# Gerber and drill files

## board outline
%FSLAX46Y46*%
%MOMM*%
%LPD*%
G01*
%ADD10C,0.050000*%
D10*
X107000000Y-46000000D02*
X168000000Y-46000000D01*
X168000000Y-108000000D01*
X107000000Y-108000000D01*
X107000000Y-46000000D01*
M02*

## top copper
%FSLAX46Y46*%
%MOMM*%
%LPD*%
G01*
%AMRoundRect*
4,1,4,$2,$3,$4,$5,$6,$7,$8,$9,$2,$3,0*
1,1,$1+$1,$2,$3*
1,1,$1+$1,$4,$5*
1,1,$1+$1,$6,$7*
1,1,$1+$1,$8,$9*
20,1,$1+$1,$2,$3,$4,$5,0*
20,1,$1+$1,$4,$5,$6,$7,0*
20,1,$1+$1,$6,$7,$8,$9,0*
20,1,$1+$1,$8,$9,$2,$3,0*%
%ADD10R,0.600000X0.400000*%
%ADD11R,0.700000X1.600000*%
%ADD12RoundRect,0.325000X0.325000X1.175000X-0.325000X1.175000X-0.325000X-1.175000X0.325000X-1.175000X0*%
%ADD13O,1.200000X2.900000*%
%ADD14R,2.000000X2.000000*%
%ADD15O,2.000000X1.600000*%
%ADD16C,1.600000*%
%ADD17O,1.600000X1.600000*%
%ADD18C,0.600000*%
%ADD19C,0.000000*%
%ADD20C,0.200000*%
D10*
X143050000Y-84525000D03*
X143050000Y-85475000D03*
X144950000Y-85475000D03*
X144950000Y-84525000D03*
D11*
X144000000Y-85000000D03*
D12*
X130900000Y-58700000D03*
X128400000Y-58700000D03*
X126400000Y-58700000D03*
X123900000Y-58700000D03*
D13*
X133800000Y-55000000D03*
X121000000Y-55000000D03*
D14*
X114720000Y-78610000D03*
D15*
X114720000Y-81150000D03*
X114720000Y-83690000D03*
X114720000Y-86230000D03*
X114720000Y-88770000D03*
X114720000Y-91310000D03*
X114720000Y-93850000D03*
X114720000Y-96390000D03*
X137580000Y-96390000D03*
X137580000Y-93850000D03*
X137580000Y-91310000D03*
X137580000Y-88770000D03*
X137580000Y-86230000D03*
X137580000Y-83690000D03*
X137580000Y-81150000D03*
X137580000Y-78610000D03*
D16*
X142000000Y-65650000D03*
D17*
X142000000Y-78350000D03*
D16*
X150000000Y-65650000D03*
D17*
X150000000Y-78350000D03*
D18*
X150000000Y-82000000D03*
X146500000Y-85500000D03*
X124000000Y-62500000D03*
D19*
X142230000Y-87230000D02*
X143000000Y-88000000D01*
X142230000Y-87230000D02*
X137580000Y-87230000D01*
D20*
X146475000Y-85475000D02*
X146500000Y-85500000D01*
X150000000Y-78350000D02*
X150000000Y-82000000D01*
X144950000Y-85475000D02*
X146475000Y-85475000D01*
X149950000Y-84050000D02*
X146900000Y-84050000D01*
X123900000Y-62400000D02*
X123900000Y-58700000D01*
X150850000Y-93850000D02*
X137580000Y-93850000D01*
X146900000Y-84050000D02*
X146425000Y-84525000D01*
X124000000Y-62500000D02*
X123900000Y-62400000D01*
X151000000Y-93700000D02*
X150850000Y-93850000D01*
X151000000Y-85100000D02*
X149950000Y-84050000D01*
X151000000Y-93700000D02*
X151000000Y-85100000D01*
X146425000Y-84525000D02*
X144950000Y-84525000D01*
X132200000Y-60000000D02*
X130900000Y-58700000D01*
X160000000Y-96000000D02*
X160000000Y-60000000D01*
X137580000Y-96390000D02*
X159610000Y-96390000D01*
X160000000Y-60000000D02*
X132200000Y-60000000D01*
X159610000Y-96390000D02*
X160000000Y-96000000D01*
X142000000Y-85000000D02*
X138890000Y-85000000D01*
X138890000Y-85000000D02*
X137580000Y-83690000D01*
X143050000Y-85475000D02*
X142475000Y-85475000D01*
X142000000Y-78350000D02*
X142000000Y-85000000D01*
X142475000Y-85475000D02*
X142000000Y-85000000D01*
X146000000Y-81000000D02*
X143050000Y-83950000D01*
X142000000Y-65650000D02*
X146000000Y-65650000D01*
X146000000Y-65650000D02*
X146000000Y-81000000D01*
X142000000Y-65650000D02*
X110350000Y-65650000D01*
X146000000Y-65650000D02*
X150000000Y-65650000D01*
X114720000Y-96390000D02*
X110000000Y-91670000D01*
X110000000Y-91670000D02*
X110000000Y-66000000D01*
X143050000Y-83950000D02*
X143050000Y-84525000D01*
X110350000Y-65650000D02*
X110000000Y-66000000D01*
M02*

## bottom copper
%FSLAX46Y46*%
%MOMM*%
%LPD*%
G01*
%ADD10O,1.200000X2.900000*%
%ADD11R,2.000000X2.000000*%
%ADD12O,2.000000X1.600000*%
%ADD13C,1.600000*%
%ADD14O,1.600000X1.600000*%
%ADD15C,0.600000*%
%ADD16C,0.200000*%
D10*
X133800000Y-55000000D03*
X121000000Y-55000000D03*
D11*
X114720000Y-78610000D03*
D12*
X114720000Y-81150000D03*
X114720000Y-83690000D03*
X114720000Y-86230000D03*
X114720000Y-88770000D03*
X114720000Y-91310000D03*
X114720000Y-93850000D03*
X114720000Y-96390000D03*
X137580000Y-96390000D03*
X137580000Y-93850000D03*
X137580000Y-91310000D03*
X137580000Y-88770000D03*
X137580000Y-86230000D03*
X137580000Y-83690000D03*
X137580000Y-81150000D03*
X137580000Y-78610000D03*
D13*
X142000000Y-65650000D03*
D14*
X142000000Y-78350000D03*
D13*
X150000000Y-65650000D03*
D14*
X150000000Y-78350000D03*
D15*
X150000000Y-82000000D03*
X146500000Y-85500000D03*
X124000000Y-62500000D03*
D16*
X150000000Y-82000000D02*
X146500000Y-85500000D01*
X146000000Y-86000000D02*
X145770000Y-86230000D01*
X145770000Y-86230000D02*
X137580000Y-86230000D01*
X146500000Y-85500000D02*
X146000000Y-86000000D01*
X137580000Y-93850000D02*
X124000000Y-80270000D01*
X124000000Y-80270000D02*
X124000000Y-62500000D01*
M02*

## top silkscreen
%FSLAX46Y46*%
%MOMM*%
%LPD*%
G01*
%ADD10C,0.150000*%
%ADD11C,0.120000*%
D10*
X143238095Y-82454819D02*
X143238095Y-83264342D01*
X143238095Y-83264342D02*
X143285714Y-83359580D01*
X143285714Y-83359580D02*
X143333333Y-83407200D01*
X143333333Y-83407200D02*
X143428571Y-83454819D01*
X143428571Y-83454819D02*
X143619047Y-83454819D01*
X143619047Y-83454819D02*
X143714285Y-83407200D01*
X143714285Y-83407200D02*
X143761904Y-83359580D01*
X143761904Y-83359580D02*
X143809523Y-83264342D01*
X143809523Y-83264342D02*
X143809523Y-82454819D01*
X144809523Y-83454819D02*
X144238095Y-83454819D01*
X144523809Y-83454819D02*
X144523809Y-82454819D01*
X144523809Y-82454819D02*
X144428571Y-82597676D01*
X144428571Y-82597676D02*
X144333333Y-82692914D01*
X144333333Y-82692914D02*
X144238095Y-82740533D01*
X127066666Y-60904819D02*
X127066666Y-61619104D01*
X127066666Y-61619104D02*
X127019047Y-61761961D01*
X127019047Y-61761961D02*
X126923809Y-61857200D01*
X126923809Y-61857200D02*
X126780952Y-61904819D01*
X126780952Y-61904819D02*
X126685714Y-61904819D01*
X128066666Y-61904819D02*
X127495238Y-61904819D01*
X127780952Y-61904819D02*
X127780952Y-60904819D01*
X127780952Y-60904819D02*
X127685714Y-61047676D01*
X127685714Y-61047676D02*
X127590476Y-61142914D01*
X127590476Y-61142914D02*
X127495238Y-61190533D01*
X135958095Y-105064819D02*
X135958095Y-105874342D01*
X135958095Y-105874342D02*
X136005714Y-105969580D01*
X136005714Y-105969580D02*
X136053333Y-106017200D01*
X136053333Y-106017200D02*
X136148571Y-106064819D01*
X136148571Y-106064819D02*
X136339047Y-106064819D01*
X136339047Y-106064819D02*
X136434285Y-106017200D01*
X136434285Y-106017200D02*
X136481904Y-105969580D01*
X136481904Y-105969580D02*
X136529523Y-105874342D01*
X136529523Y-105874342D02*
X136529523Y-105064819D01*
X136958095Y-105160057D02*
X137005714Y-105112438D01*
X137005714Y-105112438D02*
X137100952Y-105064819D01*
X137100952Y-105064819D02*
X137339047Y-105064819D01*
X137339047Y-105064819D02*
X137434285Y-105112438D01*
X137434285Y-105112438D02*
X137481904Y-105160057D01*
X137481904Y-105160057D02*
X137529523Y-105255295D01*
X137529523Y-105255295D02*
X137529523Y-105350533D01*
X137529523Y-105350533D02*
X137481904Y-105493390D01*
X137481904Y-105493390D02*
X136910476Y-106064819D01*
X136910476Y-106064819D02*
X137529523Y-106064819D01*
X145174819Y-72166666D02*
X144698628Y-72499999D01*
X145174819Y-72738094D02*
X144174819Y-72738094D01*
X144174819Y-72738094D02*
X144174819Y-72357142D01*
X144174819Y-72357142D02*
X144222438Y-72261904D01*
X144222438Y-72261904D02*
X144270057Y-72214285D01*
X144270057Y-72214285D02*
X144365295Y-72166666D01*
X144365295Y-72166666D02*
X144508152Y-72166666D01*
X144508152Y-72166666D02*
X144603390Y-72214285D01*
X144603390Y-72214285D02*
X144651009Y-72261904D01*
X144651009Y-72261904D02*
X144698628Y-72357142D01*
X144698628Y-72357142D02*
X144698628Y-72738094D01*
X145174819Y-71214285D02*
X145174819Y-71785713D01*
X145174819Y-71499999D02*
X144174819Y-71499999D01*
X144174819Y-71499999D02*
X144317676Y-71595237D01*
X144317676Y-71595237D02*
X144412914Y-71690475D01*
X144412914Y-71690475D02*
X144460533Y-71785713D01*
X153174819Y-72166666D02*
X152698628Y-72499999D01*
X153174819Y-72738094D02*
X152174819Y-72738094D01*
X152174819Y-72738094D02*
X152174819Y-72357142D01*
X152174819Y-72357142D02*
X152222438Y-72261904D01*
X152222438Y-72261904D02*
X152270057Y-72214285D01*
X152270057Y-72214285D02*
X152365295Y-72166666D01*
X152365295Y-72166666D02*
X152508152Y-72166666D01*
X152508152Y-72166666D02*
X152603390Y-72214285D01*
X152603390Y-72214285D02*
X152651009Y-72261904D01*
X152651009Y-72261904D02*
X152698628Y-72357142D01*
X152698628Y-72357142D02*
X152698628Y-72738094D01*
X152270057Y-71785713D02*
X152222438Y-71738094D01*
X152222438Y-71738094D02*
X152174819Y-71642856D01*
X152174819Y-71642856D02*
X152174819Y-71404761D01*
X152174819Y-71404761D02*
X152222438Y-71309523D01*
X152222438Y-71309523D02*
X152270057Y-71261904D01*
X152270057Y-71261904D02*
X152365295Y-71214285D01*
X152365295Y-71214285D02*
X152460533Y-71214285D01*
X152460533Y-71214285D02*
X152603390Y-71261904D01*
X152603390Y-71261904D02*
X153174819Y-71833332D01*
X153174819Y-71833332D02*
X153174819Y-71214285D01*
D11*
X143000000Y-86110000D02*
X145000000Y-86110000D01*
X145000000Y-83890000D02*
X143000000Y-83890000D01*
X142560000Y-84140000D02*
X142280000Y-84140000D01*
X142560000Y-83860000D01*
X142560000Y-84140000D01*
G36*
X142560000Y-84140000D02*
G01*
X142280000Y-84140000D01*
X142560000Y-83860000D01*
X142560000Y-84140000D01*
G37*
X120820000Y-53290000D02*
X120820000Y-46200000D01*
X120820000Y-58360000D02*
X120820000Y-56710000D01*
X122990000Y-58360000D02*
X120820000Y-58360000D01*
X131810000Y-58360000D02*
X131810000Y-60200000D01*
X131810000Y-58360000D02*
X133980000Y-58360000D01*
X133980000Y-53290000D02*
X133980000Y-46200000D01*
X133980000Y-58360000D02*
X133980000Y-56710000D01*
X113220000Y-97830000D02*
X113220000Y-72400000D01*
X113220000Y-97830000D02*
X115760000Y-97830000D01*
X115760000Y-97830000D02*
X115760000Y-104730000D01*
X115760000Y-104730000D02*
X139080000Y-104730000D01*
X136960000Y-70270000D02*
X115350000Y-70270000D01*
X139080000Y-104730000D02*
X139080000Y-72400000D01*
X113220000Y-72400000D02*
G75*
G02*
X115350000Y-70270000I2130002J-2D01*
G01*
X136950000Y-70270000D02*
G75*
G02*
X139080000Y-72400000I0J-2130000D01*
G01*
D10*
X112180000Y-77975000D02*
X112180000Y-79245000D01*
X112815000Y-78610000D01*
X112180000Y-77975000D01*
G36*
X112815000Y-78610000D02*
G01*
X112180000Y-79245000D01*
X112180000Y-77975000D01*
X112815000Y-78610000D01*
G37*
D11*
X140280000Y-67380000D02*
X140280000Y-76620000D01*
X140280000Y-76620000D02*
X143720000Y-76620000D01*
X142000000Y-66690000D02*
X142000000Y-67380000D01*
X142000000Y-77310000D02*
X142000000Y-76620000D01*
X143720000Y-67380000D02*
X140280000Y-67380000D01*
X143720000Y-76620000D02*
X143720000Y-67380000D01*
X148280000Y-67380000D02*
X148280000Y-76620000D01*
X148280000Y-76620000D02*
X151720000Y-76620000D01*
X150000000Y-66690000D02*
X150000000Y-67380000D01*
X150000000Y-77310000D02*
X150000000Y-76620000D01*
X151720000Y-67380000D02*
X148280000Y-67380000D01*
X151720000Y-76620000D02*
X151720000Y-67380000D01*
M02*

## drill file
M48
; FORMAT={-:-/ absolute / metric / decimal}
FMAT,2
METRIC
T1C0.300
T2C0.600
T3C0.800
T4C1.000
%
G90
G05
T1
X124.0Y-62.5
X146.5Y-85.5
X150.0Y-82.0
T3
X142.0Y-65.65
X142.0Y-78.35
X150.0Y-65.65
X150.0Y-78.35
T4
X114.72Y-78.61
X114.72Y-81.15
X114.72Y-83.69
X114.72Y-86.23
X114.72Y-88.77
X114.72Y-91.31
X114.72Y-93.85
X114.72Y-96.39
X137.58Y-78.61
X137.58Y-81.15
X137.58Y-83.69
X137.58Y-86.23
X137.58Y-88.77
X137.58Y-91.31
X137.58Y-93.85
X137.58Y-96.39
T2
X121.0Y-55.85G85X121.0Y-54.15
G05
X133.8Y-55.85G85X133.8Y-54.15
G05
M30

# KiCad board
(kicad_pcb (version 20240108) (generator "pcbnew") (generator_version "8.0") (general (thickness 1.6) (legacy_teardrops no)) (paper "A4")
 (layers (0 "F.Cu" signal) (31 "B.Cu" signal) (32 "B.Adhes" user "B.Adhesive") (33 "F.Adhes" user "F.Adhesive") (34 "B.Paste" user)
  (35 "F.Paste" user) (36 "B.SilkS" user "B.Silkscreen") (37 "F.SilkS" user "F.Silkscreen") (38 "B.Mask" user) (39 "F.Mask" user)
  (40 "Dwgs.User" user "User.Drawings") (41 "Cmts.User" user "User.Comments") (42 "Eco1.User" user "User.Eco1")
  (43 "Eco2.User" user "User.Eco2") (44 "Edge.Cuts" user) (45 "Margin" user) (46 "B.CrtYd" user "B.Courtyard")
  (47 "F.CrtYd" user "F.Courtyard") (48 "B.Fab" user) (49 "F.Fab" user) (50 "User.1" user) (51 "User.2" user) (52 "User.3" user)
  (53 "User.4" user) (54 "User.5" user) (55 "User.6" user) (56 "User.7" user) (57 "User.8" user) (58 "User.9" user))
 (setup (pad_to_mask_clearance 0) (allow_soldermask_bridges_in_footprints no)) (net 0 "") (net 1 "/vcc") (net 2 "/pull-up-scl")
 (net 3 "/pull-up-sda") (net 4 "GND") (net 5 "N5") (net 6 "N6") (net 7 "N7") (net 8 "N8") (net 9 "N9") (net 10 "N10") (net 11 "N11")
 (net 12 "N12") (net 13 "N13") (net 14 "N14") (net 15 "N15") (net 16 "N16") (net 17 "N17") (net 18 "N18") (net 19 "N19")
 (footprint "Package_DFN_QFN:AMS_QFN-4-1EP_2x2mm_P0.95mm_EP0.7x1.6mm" (layer "F.Cu") (at 144 85)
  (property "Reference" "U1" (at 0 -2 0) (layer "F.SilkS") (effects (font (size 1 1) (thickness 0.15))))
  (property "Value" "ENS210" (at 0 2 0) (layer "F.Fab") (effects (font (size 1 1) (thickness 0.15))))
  (fp_line (start -1 1.11) (end 1 1.11) (stroke (width 0.12) (type solid)) (layer "F.SilkS"))
  (fp_line (start 1 -1.11) (end -1 -1.11) (stroke (width 0.12) (type solid)) (layer "F.SilkS"))
  (fp_poly
   (pts (xy -1.44 -0.86) (xy -1.72 -0.86) (xy -1.44 -1.14) (xy -1.44 -0.86)) (stroke (width 0.12) (type solid)) (fill solid)
   (layer "F.SilkS"))
  (pad "" smd rect (at 0 0) (size 0.35 0.8) (layers "F.Paste"))
  (pad "1" smd rect (at -0.95 -0.475) (size 0.6 0.4) (layers "F.Cu" "F.Paste" "F.Mask") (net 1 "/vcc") (solder_paste_margin -0.05))
  (pad "2" smd rect (at -0.95 0.475) (size 0.6 0.4) (layers "F.Cu" "F.Paste" "F.Mask") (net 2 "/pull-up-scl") (solder_paste_margin -0.05))
  (pad "3" smd rect (at 0.95 0.475) (size 0.6 0.4) (layers "F.Cu" "F.Paste" "F.Mask") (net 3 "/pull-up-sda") (solder_paste_margin -0.05))
  (pad "4" smd rect (at 0.95 -0.475) (size 0.6 0.4) (layers "F.Cu" "F.Paste" "F.Mask") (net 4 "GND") (solder_paste_margin -0.05))
  (pad "5" smd rect (at 0 0) (size 0.7 1.6) (layers "F.Cu" "F.Mask") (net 4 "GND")))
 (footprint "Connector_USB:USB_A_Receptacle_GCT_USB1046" (layer "F.Cu") (at 127.4 51.45 180)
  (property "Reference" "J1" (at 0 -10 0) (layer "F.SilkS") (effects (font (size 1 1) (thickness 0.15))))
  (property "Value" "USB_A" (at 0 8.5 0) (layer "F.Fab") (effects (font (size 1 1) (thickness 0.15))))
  (fp_line (start 6.58 -1.84) (end 6.58 5.25) (stroke (width 0.12) (type default)) (layer "F.SilkS"))
  (fp_line (start 6.58 -6.91) (end 6.58 -5.26) (stroke (width 0.12) (type default)) (layer "F.SilkS"))
  (fp_line (start 4.41 -6.91) (end 6.58 -6.91) (stroke (width 0.12) (type default)) (layer "F.SilkS"))
  (fp_line (start -4.41 -6.91) (end -4.41 -8.75) (stroke (width 0.12) (type default)) (layer "F.SilkS"))
  (fp_line (start -4.41 -6.91) (end -6.58 -6.91) (stroke (width 0.12) (type default)) (layer "F.SilkS"))
  (fp_line (start -6.58 -1.84) (end -6.58 5.25) (stroke (width 0.12) (type default)) (layer "F.SilkS"))
  (fp_line (start -6.58 -6.91) (end -6.58 -5.26) (stroke (width 0.12) (type default)) (layer "F.SilkS"))
  (pad "" smd oval (at -6.4 -3.55 180) (size 1.2 2.9) (layers "F.Paste") (thermal_bridge_angle 45))
  (pad "" smd oval (at 6.4 -3.55 180) (size 1.2 2.9) (layers "F.Paste") (thermal_bridge_angle 45))
  (pad "1" smd roundrect (at -3.5 -7.25 180) (size 1.3 3) (layers "F.Cu" "F.Paste" "F.Mask") (roundrect_rratio 0.25) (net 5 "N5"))
  (pad "2" smd roundrect (at -1 -7.25 180) (size 1.3 3) (layers "F.Cu" "F.Paste" "F.Mask") (roundrect_rratio 0.25) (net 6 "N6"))
  (pad "3" smd roundrect (at 1 -7.25 180) (size 1.3 3) (layers "F.Cu" "F.Paste" "F.Mask") (roundrect_rratio 0.25) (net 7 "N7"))
  (pad "4" smd roundrect (at 3.5 -7.25 180) (size 1.3 3) (layers "F.Cu" "F.Paste" "F.Mask") (roundrect_rratio 0.25) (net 4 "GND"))
  (pad "5" thru_hole oval (at -6.4 -3.55 180) (size 1.2 2.9) (drill oval 0.6 2.3) (layers "*.Cu" "*.Mask") (remove_unused_layers no)
   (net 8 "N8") (thermal_bridge_angle 45))
  (pad "5" thru_hole oval (at 6.4 -3.55 180) (size 1.2 2.9) (drill oval 0.6 2.3) (layers "*.Cu" "*.Mask") (remove_unused_layers no)
   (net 8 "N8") (thermal_bridge_angle 45)))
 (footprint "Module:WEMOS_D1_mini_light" (layer "F.Cu") (at 114.72 78.61)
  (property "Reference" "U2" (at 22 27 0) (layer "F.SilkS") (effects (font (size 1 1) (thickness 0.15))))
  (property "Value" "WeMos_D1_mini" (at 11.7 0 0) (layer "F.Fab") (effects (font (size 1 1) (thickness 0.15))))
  (fp_line (start -1.5 19.22) (end -1.5 -6.21) (stroke (width 0.12) (type solid)) (layer "F.SilkS"))
  (fp_line (start -1.5 19.22) (end 1.04 19.22) (stroke (width 0.12) (type solid)) (layer "F.SilkS"))
  (fp_line (start 1.04 19.22) (end 1.04 26.12) (stroke (width 0.12) (type solid)) (layer "F.SilkS"))
  (fp_line (start 1.04 26.12) (end 24.36 26.12) (stroke (width 0.12) (type solid)) (layer "F.SilkS"))
  (fp_line (start 22.24 -8.34) (end 0.63 -8.34) (stroke (width 0.12) (type solid)) (layer "F.SilkS"))
  (fp_line (start 24.36 26.12) (end 24.36 -6.21) (stroke (width 0.12) (type solid)) (layer "F.SilkS"))
  (fp_arc (start -1.5 -6.21) (mid -0.876137 -7.716137) (end 0.63 -8.34) (stroke (width 0.12) (type solid)) (layer "F.SilkS"))
  (fp_arc (start 22.23 -8.34) (mid 23.736137 -7.716137) (end 24.36 -6.21) (stroke (width 0.12) (type solid)) (layer "F.SilkS"))
  (fp_poly (pts (xy -2.54 -0.635) (xy -2.54 0.635) (xy -1.905 0)) (stroke (width 0.15) (type solid)) (fill solid) (layer "F.SilkS"))
  (pad "1" thru_hole rect (at 0 0) (size 2 2) (drill 1) (layers "*.Cu" "*.Mask") (remove_unused_layers no) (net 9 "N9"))
  (pad "2" thru_hole oval (at 0 2.54) (size 2 1.6) (drill 1) (layers "*.Cu" "*.Mask") (remove_unused_layers no) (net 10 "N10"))
  (pad "3" thru_hole oval (at 0 5.08) (size 2 1.6) (drill 1) (layers "*.Cu" "*.Mask") (remove_unused_layers no) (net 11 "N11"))
  (pad "4" thru_hole oval (at 0 7.62) (size 2 1.6) (drill 1) (layers "*.Cu" "*.Mask") (remove_unused_layers no) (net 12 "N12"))
  (pad "5" thru_hole oval (at 0 10.16) (size 2 1.6) (drill 1) (layers "*.Cu" "*.Mask") (remove_unused_layers no) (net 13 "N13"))
  (pad "6" thru_hole oval (at 0 12.7) (size 2 1.6) (drill 1) (layers "*.Cu" "*.Mask") (remove_unused_layers no) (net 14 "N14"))
  (pad "7" thru_hole oval (at 0 15.24) (size 2 1.6) (drill 1) (layers "*.Cu" "*.Mask") (remove_unused_layers no) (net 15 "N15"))
  (pad "8" thru_hole oval (at 0 17.78) (size 2 1.6) (drill 1) (layers "*.Cu" "*.Mask") (remove_unused_layers no) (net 1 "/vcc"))
  (pad "9" thru_hole oval (at 22.86 17.78) (size 2 1.6) (drill 1) (layers "*.Cu" "*.Mask") (remove_unused_layers no) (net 5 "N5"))
  (pad "10" thru_hole oval (at 22.86 15.24) (size 2 1.6) (drill 1) (layers "*.Cu" "*.Mask") (remove_unused_layers no) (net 4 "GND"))
  (pad "11" thru_hole oval (at 22.86 12.7) (size 2 1.6) (drill 1) (layers "*.Cu" "*.Mask") (remove_unused_layers no) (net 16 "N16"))
  (pad "12" thru_hole oval (at 22.86 10.16) (size 2 1.6) (drill 1) (layers "*.Cu" "*.Mask") (remove_unused_layers no) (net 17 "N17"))
  (pad "13" thru_hole oval (at 22.86 7.62) (size 2 1.6) (drill 1) (layers "*.Cu" "*.Mask") (remove_unused_layers no) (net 3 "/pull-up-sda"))
  (pad "14" thru_hole oval (at 22.86 5.08) (size 2 1.6) (drill 1) (layers "*.Cu" "*.Mask") (remove_unused_layers no) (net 2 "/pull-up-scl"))
  (pad "15" thru_hole oval (at 22.86 2.54) (size 2 1.6) (drill 1) (layers "*.Cu" "*.Mask") (remove_unused_layers no) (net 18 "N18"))
  (pad "16" thru_hole oval (at 22.86 0) (size 2 1.6) (drill 1) (layers "*.Cu" "*.Mask") (remove_unused_layers no) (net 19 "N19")))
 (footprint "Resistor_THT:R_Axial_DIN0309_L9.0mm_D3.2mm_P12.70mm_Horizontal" (layer "F.Cu") (at 142 65.65 -90)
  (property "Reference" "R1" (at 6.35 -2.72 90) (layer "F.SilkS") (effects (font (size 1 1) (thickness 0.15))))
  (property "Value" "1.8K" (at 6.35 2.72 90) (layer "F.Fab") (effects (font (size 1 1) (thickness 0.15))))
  (fp_line (start 1.73 1.72) (end 10.97 1.72) (stroke (width 0.12) (type solid)) (layer "F.SilkS"))
  (fp_line (start 10.97 1.72) (end 10.97 -1.72) (stroke (width 0.12) (type solid)) (layer "F.SilkS"))
  (fp_line (start 1.04 0) (end 1.73 0) (stroke (width 0.12) (type solid)) (layer "F.SilkS"))
  (fp_line (start 11.66 0) (end 10.97 0) (stroke (width 0.12) (type solid)) (layer "F.SilkS"))
  (fp_line (start 1.73 -1.72) (end 1.73 1.72) (stroke (width 0.12) (type solid)) (layer "F.SilkS"))
  (fp_line (start 10.97 -1.72) (end 1.73 -1.72) (stroke (width 0.12) (type solid)) (layer "F.SilkS"))
  (pad "1" thru_hole circle (at 0 0 270) (size 1.6 1.6) (drill 0.8) (layers "*.Cu" "*.Mask") (remove_unused_layers no) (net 1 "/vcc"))
  (pad "2" thru_hole oval (at 12.7 0 270) (size 1.6 1.6) (drill 0.8) (layers "*.Cu" "*.Mask") (remove_unused_layers no)
   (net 2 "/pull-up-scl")))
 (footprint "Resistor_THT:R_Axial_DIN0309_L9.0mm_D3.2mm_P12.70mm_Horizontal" (layer "F.Cu") (at 150 65.65 -90)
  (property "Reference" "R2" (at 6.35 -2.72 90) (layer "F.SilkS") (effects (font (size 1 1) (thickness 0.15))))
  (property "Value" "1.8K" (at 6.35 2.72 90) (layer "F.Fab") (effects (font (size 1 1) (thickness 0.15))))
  (fp_line (start 1.73 1.72) (end 10.97 1.72) (stroke (width 0.12) (type solid)) (layer "F.SilkS"))
  (fp_line (start 10.97 1.72) (end 10.97 -1.72) (stroke (width 0.12) (type solid)) (layer "F.SilkS"))
  (fp_line (start 1.04 0) (end 1.73 0) (stroke (width 0.12) (type solid)) (layer "F.SilkS"))
  (fp_line (start 11.66 0) (end 10.97 0) (stroke (width 0.12) (type solid)) (layer "F.SilkS"))
  (fp_line (start 1.73 -1.72) (end 1.73 1.72) (stroke (width 0.12) (type solid)) (layer "F.SilkS"))
  (fp_line (start 10.97 -1.72) (end 1.73 -1.72) (stroke (width 0.12) (type solid)) (layer "F.SilkS"))
  (pad "1" thru_hole circle (at 0 0 270) (size 1.6 1.6) (drill 0.8) (layers "*.Cu" "*.Mask") (remove_unused_layers no) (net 1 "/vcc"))
  (pad "2" thru_hole oval (at 12.7 0 270) (size 1.6 1.6) (drill 0.8) (layers "*.Cu" "*.Mask") (remove_unused_layers no)
   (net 3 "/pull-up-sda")))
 (gr_rect (start 107 46) (end 168 108) (stroke (width 0.05) (type default)) (fill none) (layer "Edge.Cuts"))
 (segment (start 142.23 87.23) (end 143 88) (width 0) (layer "F.Cu") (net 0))
 (segment (start 142.23 87.23) (end 137.58 87.23) (width 0) (layer "F.Cu") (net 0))
 (segment (start 146.475 85.475) (end 146.5 85.5) (width 0.2) (layer "F.Cu") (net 3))
 (segment (start 150 78.35) (end 150 82) (width 0.2) (layer "F.Cu") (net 3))
 (segment (start 144.95 85.475) (end 146.475 85.475) (width 0.2) (layer "F.Cu") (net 3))
 (via (at 150 82) (size 0.6) (drill 0.3) (layers "F.Cu" "B.Cu") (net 3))
 (via (at 146.5 85.5) (size 0.6) (drill 0.3) (layers "F.Cu" "B.Cu") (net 3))
 (segment (start 150 82) (end 146.5 85.5) (width 0.2) (layer "B.Cu") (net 3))
 (segment (start 146 86) (end 145.77 86.23) (width 0.2) (layer "B.Cu") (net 3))
 (segment (start 145.77 86.23) (end 137.58 86.23) (width 0.2) (layer "B.Cu") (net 3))
 (segment (start 146.5 85.5) (end 146 86) (width 0.2) (layer "B.Cu") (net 3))
 (segment (start 149.95 84.05) (end 146.9 84.05) (width 0.2) (layer "F.Cu") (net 4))
 (segment (start 123.9 62.4) (end 123.9 58.7) (width 0.2) (layer "F.Cu") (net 4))
 (segment (start 150.85 93.85) (end 137.58 93.85) (width 0.2) (layer "F.Cu") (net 4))
 (segment (start 146.9 84.05) (end 146.425 84.525) (width 0.2) (layer "F.Cu") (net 4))
 (segment (start 124 62.5) (end 123.9 62.4) (width 0.2) (layer "F.Cu") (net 4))
 (segment (start 151 93.7) (end 150.85 93.85) (width 0.2) (layer "F.Cu") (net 4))
 (segment (start 151 85.1) (end 149.95 84.05) (width 0.2) (layer "F.Cu") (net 4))
 (segment (start 151 93.7) (end 151 85.1) (width 0.2) (layer "F.Cu") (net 4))
 (segment (start 146.425 84.525) (end 144.95 84.525) (width 0.2) (layer "F.Cu") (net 4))
 (via (at 124 62.5) (size 0.6) (drill 0.3) (layers "F.Cu" "B.Cu") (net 4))
 (segment (start 137.58 93.85) (end 124 80.27) (width 0.2) (layer "B.Cu") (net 4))
 (segment (start 124 80.27) (end 124 62.5) (width 0.2) (layer "B.Cu") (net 4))
 (segment (start 132.2 60) (end 130.9 58.7) (width 0.2) (layer "F.Cu") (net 5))
 (segment (start 160 96) (end 160 60) (width 0.2) (layer "F.Cu") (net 5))
 (segment (start 137.58 96.39) (end 159.61 96.39) (width 0.2) (layer "F.Cu") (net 5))
 (segment (start 160 60) (end 132.2 60) (width 0.2) (layer "F.Cu") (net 5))
 (segment (start 159.61 96.39) (end 160 96) (width 0.2) (layer "F.Cu") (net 5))
 (segment (start 142 85) (end 138.89 85) (width 0.2) (layer "F.Cu") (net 2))
 (segment (start 138.89 85) (end 137.58 83.69) (width 0.2) (layer "F.Cu") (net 2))
 (segment (start 143.05 85.475) (end 142.475 85.475) (width 0.2) (layer "F.Cu") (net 2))
 (segment (start 142 78.35) (end 142 85) (width 0.2) (layer "F.Cu") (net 2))
 (segment (start 142.475 85.475) (end 142 85) (width 0.2) (layer "F.Cu") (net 2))
 (segment (start 146 81) (end 143.05 83.95) (width 0.2) (layer "F.Cu") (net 1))
 (segment (start 142 65.65) (end 146 65.65) (width 0.2) (layer "F.Cu") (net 1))
 (segment (start 146 65.65) (end 146 81) (width 0.2) (layer "F.Cu") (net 1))
 (segment (start 142 65.65) (end 110.35 65.65) (width 0.2) (layer "F.Cu") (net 1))
 (segment (start 146 65.65) (end 150 65.65) (width 0.2) (layer "F.Cu") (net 1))
 (segment (start 114.72 96.39) (end 110 91.67) (width 0.2) (layer "F.Cu") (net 1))
 (segment (start 110 91.67) (end 110 66) (width 0.2) (layer "F.Cu") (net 1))
 (segment (start 143.05 83.95) (end 143.05 84.525) (width 0.2) (layer "F.Cu") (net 1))
 (segment (start 110.35 65.65) (end 110 66) (width 0.2) (layer "F.Cu") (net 1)))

